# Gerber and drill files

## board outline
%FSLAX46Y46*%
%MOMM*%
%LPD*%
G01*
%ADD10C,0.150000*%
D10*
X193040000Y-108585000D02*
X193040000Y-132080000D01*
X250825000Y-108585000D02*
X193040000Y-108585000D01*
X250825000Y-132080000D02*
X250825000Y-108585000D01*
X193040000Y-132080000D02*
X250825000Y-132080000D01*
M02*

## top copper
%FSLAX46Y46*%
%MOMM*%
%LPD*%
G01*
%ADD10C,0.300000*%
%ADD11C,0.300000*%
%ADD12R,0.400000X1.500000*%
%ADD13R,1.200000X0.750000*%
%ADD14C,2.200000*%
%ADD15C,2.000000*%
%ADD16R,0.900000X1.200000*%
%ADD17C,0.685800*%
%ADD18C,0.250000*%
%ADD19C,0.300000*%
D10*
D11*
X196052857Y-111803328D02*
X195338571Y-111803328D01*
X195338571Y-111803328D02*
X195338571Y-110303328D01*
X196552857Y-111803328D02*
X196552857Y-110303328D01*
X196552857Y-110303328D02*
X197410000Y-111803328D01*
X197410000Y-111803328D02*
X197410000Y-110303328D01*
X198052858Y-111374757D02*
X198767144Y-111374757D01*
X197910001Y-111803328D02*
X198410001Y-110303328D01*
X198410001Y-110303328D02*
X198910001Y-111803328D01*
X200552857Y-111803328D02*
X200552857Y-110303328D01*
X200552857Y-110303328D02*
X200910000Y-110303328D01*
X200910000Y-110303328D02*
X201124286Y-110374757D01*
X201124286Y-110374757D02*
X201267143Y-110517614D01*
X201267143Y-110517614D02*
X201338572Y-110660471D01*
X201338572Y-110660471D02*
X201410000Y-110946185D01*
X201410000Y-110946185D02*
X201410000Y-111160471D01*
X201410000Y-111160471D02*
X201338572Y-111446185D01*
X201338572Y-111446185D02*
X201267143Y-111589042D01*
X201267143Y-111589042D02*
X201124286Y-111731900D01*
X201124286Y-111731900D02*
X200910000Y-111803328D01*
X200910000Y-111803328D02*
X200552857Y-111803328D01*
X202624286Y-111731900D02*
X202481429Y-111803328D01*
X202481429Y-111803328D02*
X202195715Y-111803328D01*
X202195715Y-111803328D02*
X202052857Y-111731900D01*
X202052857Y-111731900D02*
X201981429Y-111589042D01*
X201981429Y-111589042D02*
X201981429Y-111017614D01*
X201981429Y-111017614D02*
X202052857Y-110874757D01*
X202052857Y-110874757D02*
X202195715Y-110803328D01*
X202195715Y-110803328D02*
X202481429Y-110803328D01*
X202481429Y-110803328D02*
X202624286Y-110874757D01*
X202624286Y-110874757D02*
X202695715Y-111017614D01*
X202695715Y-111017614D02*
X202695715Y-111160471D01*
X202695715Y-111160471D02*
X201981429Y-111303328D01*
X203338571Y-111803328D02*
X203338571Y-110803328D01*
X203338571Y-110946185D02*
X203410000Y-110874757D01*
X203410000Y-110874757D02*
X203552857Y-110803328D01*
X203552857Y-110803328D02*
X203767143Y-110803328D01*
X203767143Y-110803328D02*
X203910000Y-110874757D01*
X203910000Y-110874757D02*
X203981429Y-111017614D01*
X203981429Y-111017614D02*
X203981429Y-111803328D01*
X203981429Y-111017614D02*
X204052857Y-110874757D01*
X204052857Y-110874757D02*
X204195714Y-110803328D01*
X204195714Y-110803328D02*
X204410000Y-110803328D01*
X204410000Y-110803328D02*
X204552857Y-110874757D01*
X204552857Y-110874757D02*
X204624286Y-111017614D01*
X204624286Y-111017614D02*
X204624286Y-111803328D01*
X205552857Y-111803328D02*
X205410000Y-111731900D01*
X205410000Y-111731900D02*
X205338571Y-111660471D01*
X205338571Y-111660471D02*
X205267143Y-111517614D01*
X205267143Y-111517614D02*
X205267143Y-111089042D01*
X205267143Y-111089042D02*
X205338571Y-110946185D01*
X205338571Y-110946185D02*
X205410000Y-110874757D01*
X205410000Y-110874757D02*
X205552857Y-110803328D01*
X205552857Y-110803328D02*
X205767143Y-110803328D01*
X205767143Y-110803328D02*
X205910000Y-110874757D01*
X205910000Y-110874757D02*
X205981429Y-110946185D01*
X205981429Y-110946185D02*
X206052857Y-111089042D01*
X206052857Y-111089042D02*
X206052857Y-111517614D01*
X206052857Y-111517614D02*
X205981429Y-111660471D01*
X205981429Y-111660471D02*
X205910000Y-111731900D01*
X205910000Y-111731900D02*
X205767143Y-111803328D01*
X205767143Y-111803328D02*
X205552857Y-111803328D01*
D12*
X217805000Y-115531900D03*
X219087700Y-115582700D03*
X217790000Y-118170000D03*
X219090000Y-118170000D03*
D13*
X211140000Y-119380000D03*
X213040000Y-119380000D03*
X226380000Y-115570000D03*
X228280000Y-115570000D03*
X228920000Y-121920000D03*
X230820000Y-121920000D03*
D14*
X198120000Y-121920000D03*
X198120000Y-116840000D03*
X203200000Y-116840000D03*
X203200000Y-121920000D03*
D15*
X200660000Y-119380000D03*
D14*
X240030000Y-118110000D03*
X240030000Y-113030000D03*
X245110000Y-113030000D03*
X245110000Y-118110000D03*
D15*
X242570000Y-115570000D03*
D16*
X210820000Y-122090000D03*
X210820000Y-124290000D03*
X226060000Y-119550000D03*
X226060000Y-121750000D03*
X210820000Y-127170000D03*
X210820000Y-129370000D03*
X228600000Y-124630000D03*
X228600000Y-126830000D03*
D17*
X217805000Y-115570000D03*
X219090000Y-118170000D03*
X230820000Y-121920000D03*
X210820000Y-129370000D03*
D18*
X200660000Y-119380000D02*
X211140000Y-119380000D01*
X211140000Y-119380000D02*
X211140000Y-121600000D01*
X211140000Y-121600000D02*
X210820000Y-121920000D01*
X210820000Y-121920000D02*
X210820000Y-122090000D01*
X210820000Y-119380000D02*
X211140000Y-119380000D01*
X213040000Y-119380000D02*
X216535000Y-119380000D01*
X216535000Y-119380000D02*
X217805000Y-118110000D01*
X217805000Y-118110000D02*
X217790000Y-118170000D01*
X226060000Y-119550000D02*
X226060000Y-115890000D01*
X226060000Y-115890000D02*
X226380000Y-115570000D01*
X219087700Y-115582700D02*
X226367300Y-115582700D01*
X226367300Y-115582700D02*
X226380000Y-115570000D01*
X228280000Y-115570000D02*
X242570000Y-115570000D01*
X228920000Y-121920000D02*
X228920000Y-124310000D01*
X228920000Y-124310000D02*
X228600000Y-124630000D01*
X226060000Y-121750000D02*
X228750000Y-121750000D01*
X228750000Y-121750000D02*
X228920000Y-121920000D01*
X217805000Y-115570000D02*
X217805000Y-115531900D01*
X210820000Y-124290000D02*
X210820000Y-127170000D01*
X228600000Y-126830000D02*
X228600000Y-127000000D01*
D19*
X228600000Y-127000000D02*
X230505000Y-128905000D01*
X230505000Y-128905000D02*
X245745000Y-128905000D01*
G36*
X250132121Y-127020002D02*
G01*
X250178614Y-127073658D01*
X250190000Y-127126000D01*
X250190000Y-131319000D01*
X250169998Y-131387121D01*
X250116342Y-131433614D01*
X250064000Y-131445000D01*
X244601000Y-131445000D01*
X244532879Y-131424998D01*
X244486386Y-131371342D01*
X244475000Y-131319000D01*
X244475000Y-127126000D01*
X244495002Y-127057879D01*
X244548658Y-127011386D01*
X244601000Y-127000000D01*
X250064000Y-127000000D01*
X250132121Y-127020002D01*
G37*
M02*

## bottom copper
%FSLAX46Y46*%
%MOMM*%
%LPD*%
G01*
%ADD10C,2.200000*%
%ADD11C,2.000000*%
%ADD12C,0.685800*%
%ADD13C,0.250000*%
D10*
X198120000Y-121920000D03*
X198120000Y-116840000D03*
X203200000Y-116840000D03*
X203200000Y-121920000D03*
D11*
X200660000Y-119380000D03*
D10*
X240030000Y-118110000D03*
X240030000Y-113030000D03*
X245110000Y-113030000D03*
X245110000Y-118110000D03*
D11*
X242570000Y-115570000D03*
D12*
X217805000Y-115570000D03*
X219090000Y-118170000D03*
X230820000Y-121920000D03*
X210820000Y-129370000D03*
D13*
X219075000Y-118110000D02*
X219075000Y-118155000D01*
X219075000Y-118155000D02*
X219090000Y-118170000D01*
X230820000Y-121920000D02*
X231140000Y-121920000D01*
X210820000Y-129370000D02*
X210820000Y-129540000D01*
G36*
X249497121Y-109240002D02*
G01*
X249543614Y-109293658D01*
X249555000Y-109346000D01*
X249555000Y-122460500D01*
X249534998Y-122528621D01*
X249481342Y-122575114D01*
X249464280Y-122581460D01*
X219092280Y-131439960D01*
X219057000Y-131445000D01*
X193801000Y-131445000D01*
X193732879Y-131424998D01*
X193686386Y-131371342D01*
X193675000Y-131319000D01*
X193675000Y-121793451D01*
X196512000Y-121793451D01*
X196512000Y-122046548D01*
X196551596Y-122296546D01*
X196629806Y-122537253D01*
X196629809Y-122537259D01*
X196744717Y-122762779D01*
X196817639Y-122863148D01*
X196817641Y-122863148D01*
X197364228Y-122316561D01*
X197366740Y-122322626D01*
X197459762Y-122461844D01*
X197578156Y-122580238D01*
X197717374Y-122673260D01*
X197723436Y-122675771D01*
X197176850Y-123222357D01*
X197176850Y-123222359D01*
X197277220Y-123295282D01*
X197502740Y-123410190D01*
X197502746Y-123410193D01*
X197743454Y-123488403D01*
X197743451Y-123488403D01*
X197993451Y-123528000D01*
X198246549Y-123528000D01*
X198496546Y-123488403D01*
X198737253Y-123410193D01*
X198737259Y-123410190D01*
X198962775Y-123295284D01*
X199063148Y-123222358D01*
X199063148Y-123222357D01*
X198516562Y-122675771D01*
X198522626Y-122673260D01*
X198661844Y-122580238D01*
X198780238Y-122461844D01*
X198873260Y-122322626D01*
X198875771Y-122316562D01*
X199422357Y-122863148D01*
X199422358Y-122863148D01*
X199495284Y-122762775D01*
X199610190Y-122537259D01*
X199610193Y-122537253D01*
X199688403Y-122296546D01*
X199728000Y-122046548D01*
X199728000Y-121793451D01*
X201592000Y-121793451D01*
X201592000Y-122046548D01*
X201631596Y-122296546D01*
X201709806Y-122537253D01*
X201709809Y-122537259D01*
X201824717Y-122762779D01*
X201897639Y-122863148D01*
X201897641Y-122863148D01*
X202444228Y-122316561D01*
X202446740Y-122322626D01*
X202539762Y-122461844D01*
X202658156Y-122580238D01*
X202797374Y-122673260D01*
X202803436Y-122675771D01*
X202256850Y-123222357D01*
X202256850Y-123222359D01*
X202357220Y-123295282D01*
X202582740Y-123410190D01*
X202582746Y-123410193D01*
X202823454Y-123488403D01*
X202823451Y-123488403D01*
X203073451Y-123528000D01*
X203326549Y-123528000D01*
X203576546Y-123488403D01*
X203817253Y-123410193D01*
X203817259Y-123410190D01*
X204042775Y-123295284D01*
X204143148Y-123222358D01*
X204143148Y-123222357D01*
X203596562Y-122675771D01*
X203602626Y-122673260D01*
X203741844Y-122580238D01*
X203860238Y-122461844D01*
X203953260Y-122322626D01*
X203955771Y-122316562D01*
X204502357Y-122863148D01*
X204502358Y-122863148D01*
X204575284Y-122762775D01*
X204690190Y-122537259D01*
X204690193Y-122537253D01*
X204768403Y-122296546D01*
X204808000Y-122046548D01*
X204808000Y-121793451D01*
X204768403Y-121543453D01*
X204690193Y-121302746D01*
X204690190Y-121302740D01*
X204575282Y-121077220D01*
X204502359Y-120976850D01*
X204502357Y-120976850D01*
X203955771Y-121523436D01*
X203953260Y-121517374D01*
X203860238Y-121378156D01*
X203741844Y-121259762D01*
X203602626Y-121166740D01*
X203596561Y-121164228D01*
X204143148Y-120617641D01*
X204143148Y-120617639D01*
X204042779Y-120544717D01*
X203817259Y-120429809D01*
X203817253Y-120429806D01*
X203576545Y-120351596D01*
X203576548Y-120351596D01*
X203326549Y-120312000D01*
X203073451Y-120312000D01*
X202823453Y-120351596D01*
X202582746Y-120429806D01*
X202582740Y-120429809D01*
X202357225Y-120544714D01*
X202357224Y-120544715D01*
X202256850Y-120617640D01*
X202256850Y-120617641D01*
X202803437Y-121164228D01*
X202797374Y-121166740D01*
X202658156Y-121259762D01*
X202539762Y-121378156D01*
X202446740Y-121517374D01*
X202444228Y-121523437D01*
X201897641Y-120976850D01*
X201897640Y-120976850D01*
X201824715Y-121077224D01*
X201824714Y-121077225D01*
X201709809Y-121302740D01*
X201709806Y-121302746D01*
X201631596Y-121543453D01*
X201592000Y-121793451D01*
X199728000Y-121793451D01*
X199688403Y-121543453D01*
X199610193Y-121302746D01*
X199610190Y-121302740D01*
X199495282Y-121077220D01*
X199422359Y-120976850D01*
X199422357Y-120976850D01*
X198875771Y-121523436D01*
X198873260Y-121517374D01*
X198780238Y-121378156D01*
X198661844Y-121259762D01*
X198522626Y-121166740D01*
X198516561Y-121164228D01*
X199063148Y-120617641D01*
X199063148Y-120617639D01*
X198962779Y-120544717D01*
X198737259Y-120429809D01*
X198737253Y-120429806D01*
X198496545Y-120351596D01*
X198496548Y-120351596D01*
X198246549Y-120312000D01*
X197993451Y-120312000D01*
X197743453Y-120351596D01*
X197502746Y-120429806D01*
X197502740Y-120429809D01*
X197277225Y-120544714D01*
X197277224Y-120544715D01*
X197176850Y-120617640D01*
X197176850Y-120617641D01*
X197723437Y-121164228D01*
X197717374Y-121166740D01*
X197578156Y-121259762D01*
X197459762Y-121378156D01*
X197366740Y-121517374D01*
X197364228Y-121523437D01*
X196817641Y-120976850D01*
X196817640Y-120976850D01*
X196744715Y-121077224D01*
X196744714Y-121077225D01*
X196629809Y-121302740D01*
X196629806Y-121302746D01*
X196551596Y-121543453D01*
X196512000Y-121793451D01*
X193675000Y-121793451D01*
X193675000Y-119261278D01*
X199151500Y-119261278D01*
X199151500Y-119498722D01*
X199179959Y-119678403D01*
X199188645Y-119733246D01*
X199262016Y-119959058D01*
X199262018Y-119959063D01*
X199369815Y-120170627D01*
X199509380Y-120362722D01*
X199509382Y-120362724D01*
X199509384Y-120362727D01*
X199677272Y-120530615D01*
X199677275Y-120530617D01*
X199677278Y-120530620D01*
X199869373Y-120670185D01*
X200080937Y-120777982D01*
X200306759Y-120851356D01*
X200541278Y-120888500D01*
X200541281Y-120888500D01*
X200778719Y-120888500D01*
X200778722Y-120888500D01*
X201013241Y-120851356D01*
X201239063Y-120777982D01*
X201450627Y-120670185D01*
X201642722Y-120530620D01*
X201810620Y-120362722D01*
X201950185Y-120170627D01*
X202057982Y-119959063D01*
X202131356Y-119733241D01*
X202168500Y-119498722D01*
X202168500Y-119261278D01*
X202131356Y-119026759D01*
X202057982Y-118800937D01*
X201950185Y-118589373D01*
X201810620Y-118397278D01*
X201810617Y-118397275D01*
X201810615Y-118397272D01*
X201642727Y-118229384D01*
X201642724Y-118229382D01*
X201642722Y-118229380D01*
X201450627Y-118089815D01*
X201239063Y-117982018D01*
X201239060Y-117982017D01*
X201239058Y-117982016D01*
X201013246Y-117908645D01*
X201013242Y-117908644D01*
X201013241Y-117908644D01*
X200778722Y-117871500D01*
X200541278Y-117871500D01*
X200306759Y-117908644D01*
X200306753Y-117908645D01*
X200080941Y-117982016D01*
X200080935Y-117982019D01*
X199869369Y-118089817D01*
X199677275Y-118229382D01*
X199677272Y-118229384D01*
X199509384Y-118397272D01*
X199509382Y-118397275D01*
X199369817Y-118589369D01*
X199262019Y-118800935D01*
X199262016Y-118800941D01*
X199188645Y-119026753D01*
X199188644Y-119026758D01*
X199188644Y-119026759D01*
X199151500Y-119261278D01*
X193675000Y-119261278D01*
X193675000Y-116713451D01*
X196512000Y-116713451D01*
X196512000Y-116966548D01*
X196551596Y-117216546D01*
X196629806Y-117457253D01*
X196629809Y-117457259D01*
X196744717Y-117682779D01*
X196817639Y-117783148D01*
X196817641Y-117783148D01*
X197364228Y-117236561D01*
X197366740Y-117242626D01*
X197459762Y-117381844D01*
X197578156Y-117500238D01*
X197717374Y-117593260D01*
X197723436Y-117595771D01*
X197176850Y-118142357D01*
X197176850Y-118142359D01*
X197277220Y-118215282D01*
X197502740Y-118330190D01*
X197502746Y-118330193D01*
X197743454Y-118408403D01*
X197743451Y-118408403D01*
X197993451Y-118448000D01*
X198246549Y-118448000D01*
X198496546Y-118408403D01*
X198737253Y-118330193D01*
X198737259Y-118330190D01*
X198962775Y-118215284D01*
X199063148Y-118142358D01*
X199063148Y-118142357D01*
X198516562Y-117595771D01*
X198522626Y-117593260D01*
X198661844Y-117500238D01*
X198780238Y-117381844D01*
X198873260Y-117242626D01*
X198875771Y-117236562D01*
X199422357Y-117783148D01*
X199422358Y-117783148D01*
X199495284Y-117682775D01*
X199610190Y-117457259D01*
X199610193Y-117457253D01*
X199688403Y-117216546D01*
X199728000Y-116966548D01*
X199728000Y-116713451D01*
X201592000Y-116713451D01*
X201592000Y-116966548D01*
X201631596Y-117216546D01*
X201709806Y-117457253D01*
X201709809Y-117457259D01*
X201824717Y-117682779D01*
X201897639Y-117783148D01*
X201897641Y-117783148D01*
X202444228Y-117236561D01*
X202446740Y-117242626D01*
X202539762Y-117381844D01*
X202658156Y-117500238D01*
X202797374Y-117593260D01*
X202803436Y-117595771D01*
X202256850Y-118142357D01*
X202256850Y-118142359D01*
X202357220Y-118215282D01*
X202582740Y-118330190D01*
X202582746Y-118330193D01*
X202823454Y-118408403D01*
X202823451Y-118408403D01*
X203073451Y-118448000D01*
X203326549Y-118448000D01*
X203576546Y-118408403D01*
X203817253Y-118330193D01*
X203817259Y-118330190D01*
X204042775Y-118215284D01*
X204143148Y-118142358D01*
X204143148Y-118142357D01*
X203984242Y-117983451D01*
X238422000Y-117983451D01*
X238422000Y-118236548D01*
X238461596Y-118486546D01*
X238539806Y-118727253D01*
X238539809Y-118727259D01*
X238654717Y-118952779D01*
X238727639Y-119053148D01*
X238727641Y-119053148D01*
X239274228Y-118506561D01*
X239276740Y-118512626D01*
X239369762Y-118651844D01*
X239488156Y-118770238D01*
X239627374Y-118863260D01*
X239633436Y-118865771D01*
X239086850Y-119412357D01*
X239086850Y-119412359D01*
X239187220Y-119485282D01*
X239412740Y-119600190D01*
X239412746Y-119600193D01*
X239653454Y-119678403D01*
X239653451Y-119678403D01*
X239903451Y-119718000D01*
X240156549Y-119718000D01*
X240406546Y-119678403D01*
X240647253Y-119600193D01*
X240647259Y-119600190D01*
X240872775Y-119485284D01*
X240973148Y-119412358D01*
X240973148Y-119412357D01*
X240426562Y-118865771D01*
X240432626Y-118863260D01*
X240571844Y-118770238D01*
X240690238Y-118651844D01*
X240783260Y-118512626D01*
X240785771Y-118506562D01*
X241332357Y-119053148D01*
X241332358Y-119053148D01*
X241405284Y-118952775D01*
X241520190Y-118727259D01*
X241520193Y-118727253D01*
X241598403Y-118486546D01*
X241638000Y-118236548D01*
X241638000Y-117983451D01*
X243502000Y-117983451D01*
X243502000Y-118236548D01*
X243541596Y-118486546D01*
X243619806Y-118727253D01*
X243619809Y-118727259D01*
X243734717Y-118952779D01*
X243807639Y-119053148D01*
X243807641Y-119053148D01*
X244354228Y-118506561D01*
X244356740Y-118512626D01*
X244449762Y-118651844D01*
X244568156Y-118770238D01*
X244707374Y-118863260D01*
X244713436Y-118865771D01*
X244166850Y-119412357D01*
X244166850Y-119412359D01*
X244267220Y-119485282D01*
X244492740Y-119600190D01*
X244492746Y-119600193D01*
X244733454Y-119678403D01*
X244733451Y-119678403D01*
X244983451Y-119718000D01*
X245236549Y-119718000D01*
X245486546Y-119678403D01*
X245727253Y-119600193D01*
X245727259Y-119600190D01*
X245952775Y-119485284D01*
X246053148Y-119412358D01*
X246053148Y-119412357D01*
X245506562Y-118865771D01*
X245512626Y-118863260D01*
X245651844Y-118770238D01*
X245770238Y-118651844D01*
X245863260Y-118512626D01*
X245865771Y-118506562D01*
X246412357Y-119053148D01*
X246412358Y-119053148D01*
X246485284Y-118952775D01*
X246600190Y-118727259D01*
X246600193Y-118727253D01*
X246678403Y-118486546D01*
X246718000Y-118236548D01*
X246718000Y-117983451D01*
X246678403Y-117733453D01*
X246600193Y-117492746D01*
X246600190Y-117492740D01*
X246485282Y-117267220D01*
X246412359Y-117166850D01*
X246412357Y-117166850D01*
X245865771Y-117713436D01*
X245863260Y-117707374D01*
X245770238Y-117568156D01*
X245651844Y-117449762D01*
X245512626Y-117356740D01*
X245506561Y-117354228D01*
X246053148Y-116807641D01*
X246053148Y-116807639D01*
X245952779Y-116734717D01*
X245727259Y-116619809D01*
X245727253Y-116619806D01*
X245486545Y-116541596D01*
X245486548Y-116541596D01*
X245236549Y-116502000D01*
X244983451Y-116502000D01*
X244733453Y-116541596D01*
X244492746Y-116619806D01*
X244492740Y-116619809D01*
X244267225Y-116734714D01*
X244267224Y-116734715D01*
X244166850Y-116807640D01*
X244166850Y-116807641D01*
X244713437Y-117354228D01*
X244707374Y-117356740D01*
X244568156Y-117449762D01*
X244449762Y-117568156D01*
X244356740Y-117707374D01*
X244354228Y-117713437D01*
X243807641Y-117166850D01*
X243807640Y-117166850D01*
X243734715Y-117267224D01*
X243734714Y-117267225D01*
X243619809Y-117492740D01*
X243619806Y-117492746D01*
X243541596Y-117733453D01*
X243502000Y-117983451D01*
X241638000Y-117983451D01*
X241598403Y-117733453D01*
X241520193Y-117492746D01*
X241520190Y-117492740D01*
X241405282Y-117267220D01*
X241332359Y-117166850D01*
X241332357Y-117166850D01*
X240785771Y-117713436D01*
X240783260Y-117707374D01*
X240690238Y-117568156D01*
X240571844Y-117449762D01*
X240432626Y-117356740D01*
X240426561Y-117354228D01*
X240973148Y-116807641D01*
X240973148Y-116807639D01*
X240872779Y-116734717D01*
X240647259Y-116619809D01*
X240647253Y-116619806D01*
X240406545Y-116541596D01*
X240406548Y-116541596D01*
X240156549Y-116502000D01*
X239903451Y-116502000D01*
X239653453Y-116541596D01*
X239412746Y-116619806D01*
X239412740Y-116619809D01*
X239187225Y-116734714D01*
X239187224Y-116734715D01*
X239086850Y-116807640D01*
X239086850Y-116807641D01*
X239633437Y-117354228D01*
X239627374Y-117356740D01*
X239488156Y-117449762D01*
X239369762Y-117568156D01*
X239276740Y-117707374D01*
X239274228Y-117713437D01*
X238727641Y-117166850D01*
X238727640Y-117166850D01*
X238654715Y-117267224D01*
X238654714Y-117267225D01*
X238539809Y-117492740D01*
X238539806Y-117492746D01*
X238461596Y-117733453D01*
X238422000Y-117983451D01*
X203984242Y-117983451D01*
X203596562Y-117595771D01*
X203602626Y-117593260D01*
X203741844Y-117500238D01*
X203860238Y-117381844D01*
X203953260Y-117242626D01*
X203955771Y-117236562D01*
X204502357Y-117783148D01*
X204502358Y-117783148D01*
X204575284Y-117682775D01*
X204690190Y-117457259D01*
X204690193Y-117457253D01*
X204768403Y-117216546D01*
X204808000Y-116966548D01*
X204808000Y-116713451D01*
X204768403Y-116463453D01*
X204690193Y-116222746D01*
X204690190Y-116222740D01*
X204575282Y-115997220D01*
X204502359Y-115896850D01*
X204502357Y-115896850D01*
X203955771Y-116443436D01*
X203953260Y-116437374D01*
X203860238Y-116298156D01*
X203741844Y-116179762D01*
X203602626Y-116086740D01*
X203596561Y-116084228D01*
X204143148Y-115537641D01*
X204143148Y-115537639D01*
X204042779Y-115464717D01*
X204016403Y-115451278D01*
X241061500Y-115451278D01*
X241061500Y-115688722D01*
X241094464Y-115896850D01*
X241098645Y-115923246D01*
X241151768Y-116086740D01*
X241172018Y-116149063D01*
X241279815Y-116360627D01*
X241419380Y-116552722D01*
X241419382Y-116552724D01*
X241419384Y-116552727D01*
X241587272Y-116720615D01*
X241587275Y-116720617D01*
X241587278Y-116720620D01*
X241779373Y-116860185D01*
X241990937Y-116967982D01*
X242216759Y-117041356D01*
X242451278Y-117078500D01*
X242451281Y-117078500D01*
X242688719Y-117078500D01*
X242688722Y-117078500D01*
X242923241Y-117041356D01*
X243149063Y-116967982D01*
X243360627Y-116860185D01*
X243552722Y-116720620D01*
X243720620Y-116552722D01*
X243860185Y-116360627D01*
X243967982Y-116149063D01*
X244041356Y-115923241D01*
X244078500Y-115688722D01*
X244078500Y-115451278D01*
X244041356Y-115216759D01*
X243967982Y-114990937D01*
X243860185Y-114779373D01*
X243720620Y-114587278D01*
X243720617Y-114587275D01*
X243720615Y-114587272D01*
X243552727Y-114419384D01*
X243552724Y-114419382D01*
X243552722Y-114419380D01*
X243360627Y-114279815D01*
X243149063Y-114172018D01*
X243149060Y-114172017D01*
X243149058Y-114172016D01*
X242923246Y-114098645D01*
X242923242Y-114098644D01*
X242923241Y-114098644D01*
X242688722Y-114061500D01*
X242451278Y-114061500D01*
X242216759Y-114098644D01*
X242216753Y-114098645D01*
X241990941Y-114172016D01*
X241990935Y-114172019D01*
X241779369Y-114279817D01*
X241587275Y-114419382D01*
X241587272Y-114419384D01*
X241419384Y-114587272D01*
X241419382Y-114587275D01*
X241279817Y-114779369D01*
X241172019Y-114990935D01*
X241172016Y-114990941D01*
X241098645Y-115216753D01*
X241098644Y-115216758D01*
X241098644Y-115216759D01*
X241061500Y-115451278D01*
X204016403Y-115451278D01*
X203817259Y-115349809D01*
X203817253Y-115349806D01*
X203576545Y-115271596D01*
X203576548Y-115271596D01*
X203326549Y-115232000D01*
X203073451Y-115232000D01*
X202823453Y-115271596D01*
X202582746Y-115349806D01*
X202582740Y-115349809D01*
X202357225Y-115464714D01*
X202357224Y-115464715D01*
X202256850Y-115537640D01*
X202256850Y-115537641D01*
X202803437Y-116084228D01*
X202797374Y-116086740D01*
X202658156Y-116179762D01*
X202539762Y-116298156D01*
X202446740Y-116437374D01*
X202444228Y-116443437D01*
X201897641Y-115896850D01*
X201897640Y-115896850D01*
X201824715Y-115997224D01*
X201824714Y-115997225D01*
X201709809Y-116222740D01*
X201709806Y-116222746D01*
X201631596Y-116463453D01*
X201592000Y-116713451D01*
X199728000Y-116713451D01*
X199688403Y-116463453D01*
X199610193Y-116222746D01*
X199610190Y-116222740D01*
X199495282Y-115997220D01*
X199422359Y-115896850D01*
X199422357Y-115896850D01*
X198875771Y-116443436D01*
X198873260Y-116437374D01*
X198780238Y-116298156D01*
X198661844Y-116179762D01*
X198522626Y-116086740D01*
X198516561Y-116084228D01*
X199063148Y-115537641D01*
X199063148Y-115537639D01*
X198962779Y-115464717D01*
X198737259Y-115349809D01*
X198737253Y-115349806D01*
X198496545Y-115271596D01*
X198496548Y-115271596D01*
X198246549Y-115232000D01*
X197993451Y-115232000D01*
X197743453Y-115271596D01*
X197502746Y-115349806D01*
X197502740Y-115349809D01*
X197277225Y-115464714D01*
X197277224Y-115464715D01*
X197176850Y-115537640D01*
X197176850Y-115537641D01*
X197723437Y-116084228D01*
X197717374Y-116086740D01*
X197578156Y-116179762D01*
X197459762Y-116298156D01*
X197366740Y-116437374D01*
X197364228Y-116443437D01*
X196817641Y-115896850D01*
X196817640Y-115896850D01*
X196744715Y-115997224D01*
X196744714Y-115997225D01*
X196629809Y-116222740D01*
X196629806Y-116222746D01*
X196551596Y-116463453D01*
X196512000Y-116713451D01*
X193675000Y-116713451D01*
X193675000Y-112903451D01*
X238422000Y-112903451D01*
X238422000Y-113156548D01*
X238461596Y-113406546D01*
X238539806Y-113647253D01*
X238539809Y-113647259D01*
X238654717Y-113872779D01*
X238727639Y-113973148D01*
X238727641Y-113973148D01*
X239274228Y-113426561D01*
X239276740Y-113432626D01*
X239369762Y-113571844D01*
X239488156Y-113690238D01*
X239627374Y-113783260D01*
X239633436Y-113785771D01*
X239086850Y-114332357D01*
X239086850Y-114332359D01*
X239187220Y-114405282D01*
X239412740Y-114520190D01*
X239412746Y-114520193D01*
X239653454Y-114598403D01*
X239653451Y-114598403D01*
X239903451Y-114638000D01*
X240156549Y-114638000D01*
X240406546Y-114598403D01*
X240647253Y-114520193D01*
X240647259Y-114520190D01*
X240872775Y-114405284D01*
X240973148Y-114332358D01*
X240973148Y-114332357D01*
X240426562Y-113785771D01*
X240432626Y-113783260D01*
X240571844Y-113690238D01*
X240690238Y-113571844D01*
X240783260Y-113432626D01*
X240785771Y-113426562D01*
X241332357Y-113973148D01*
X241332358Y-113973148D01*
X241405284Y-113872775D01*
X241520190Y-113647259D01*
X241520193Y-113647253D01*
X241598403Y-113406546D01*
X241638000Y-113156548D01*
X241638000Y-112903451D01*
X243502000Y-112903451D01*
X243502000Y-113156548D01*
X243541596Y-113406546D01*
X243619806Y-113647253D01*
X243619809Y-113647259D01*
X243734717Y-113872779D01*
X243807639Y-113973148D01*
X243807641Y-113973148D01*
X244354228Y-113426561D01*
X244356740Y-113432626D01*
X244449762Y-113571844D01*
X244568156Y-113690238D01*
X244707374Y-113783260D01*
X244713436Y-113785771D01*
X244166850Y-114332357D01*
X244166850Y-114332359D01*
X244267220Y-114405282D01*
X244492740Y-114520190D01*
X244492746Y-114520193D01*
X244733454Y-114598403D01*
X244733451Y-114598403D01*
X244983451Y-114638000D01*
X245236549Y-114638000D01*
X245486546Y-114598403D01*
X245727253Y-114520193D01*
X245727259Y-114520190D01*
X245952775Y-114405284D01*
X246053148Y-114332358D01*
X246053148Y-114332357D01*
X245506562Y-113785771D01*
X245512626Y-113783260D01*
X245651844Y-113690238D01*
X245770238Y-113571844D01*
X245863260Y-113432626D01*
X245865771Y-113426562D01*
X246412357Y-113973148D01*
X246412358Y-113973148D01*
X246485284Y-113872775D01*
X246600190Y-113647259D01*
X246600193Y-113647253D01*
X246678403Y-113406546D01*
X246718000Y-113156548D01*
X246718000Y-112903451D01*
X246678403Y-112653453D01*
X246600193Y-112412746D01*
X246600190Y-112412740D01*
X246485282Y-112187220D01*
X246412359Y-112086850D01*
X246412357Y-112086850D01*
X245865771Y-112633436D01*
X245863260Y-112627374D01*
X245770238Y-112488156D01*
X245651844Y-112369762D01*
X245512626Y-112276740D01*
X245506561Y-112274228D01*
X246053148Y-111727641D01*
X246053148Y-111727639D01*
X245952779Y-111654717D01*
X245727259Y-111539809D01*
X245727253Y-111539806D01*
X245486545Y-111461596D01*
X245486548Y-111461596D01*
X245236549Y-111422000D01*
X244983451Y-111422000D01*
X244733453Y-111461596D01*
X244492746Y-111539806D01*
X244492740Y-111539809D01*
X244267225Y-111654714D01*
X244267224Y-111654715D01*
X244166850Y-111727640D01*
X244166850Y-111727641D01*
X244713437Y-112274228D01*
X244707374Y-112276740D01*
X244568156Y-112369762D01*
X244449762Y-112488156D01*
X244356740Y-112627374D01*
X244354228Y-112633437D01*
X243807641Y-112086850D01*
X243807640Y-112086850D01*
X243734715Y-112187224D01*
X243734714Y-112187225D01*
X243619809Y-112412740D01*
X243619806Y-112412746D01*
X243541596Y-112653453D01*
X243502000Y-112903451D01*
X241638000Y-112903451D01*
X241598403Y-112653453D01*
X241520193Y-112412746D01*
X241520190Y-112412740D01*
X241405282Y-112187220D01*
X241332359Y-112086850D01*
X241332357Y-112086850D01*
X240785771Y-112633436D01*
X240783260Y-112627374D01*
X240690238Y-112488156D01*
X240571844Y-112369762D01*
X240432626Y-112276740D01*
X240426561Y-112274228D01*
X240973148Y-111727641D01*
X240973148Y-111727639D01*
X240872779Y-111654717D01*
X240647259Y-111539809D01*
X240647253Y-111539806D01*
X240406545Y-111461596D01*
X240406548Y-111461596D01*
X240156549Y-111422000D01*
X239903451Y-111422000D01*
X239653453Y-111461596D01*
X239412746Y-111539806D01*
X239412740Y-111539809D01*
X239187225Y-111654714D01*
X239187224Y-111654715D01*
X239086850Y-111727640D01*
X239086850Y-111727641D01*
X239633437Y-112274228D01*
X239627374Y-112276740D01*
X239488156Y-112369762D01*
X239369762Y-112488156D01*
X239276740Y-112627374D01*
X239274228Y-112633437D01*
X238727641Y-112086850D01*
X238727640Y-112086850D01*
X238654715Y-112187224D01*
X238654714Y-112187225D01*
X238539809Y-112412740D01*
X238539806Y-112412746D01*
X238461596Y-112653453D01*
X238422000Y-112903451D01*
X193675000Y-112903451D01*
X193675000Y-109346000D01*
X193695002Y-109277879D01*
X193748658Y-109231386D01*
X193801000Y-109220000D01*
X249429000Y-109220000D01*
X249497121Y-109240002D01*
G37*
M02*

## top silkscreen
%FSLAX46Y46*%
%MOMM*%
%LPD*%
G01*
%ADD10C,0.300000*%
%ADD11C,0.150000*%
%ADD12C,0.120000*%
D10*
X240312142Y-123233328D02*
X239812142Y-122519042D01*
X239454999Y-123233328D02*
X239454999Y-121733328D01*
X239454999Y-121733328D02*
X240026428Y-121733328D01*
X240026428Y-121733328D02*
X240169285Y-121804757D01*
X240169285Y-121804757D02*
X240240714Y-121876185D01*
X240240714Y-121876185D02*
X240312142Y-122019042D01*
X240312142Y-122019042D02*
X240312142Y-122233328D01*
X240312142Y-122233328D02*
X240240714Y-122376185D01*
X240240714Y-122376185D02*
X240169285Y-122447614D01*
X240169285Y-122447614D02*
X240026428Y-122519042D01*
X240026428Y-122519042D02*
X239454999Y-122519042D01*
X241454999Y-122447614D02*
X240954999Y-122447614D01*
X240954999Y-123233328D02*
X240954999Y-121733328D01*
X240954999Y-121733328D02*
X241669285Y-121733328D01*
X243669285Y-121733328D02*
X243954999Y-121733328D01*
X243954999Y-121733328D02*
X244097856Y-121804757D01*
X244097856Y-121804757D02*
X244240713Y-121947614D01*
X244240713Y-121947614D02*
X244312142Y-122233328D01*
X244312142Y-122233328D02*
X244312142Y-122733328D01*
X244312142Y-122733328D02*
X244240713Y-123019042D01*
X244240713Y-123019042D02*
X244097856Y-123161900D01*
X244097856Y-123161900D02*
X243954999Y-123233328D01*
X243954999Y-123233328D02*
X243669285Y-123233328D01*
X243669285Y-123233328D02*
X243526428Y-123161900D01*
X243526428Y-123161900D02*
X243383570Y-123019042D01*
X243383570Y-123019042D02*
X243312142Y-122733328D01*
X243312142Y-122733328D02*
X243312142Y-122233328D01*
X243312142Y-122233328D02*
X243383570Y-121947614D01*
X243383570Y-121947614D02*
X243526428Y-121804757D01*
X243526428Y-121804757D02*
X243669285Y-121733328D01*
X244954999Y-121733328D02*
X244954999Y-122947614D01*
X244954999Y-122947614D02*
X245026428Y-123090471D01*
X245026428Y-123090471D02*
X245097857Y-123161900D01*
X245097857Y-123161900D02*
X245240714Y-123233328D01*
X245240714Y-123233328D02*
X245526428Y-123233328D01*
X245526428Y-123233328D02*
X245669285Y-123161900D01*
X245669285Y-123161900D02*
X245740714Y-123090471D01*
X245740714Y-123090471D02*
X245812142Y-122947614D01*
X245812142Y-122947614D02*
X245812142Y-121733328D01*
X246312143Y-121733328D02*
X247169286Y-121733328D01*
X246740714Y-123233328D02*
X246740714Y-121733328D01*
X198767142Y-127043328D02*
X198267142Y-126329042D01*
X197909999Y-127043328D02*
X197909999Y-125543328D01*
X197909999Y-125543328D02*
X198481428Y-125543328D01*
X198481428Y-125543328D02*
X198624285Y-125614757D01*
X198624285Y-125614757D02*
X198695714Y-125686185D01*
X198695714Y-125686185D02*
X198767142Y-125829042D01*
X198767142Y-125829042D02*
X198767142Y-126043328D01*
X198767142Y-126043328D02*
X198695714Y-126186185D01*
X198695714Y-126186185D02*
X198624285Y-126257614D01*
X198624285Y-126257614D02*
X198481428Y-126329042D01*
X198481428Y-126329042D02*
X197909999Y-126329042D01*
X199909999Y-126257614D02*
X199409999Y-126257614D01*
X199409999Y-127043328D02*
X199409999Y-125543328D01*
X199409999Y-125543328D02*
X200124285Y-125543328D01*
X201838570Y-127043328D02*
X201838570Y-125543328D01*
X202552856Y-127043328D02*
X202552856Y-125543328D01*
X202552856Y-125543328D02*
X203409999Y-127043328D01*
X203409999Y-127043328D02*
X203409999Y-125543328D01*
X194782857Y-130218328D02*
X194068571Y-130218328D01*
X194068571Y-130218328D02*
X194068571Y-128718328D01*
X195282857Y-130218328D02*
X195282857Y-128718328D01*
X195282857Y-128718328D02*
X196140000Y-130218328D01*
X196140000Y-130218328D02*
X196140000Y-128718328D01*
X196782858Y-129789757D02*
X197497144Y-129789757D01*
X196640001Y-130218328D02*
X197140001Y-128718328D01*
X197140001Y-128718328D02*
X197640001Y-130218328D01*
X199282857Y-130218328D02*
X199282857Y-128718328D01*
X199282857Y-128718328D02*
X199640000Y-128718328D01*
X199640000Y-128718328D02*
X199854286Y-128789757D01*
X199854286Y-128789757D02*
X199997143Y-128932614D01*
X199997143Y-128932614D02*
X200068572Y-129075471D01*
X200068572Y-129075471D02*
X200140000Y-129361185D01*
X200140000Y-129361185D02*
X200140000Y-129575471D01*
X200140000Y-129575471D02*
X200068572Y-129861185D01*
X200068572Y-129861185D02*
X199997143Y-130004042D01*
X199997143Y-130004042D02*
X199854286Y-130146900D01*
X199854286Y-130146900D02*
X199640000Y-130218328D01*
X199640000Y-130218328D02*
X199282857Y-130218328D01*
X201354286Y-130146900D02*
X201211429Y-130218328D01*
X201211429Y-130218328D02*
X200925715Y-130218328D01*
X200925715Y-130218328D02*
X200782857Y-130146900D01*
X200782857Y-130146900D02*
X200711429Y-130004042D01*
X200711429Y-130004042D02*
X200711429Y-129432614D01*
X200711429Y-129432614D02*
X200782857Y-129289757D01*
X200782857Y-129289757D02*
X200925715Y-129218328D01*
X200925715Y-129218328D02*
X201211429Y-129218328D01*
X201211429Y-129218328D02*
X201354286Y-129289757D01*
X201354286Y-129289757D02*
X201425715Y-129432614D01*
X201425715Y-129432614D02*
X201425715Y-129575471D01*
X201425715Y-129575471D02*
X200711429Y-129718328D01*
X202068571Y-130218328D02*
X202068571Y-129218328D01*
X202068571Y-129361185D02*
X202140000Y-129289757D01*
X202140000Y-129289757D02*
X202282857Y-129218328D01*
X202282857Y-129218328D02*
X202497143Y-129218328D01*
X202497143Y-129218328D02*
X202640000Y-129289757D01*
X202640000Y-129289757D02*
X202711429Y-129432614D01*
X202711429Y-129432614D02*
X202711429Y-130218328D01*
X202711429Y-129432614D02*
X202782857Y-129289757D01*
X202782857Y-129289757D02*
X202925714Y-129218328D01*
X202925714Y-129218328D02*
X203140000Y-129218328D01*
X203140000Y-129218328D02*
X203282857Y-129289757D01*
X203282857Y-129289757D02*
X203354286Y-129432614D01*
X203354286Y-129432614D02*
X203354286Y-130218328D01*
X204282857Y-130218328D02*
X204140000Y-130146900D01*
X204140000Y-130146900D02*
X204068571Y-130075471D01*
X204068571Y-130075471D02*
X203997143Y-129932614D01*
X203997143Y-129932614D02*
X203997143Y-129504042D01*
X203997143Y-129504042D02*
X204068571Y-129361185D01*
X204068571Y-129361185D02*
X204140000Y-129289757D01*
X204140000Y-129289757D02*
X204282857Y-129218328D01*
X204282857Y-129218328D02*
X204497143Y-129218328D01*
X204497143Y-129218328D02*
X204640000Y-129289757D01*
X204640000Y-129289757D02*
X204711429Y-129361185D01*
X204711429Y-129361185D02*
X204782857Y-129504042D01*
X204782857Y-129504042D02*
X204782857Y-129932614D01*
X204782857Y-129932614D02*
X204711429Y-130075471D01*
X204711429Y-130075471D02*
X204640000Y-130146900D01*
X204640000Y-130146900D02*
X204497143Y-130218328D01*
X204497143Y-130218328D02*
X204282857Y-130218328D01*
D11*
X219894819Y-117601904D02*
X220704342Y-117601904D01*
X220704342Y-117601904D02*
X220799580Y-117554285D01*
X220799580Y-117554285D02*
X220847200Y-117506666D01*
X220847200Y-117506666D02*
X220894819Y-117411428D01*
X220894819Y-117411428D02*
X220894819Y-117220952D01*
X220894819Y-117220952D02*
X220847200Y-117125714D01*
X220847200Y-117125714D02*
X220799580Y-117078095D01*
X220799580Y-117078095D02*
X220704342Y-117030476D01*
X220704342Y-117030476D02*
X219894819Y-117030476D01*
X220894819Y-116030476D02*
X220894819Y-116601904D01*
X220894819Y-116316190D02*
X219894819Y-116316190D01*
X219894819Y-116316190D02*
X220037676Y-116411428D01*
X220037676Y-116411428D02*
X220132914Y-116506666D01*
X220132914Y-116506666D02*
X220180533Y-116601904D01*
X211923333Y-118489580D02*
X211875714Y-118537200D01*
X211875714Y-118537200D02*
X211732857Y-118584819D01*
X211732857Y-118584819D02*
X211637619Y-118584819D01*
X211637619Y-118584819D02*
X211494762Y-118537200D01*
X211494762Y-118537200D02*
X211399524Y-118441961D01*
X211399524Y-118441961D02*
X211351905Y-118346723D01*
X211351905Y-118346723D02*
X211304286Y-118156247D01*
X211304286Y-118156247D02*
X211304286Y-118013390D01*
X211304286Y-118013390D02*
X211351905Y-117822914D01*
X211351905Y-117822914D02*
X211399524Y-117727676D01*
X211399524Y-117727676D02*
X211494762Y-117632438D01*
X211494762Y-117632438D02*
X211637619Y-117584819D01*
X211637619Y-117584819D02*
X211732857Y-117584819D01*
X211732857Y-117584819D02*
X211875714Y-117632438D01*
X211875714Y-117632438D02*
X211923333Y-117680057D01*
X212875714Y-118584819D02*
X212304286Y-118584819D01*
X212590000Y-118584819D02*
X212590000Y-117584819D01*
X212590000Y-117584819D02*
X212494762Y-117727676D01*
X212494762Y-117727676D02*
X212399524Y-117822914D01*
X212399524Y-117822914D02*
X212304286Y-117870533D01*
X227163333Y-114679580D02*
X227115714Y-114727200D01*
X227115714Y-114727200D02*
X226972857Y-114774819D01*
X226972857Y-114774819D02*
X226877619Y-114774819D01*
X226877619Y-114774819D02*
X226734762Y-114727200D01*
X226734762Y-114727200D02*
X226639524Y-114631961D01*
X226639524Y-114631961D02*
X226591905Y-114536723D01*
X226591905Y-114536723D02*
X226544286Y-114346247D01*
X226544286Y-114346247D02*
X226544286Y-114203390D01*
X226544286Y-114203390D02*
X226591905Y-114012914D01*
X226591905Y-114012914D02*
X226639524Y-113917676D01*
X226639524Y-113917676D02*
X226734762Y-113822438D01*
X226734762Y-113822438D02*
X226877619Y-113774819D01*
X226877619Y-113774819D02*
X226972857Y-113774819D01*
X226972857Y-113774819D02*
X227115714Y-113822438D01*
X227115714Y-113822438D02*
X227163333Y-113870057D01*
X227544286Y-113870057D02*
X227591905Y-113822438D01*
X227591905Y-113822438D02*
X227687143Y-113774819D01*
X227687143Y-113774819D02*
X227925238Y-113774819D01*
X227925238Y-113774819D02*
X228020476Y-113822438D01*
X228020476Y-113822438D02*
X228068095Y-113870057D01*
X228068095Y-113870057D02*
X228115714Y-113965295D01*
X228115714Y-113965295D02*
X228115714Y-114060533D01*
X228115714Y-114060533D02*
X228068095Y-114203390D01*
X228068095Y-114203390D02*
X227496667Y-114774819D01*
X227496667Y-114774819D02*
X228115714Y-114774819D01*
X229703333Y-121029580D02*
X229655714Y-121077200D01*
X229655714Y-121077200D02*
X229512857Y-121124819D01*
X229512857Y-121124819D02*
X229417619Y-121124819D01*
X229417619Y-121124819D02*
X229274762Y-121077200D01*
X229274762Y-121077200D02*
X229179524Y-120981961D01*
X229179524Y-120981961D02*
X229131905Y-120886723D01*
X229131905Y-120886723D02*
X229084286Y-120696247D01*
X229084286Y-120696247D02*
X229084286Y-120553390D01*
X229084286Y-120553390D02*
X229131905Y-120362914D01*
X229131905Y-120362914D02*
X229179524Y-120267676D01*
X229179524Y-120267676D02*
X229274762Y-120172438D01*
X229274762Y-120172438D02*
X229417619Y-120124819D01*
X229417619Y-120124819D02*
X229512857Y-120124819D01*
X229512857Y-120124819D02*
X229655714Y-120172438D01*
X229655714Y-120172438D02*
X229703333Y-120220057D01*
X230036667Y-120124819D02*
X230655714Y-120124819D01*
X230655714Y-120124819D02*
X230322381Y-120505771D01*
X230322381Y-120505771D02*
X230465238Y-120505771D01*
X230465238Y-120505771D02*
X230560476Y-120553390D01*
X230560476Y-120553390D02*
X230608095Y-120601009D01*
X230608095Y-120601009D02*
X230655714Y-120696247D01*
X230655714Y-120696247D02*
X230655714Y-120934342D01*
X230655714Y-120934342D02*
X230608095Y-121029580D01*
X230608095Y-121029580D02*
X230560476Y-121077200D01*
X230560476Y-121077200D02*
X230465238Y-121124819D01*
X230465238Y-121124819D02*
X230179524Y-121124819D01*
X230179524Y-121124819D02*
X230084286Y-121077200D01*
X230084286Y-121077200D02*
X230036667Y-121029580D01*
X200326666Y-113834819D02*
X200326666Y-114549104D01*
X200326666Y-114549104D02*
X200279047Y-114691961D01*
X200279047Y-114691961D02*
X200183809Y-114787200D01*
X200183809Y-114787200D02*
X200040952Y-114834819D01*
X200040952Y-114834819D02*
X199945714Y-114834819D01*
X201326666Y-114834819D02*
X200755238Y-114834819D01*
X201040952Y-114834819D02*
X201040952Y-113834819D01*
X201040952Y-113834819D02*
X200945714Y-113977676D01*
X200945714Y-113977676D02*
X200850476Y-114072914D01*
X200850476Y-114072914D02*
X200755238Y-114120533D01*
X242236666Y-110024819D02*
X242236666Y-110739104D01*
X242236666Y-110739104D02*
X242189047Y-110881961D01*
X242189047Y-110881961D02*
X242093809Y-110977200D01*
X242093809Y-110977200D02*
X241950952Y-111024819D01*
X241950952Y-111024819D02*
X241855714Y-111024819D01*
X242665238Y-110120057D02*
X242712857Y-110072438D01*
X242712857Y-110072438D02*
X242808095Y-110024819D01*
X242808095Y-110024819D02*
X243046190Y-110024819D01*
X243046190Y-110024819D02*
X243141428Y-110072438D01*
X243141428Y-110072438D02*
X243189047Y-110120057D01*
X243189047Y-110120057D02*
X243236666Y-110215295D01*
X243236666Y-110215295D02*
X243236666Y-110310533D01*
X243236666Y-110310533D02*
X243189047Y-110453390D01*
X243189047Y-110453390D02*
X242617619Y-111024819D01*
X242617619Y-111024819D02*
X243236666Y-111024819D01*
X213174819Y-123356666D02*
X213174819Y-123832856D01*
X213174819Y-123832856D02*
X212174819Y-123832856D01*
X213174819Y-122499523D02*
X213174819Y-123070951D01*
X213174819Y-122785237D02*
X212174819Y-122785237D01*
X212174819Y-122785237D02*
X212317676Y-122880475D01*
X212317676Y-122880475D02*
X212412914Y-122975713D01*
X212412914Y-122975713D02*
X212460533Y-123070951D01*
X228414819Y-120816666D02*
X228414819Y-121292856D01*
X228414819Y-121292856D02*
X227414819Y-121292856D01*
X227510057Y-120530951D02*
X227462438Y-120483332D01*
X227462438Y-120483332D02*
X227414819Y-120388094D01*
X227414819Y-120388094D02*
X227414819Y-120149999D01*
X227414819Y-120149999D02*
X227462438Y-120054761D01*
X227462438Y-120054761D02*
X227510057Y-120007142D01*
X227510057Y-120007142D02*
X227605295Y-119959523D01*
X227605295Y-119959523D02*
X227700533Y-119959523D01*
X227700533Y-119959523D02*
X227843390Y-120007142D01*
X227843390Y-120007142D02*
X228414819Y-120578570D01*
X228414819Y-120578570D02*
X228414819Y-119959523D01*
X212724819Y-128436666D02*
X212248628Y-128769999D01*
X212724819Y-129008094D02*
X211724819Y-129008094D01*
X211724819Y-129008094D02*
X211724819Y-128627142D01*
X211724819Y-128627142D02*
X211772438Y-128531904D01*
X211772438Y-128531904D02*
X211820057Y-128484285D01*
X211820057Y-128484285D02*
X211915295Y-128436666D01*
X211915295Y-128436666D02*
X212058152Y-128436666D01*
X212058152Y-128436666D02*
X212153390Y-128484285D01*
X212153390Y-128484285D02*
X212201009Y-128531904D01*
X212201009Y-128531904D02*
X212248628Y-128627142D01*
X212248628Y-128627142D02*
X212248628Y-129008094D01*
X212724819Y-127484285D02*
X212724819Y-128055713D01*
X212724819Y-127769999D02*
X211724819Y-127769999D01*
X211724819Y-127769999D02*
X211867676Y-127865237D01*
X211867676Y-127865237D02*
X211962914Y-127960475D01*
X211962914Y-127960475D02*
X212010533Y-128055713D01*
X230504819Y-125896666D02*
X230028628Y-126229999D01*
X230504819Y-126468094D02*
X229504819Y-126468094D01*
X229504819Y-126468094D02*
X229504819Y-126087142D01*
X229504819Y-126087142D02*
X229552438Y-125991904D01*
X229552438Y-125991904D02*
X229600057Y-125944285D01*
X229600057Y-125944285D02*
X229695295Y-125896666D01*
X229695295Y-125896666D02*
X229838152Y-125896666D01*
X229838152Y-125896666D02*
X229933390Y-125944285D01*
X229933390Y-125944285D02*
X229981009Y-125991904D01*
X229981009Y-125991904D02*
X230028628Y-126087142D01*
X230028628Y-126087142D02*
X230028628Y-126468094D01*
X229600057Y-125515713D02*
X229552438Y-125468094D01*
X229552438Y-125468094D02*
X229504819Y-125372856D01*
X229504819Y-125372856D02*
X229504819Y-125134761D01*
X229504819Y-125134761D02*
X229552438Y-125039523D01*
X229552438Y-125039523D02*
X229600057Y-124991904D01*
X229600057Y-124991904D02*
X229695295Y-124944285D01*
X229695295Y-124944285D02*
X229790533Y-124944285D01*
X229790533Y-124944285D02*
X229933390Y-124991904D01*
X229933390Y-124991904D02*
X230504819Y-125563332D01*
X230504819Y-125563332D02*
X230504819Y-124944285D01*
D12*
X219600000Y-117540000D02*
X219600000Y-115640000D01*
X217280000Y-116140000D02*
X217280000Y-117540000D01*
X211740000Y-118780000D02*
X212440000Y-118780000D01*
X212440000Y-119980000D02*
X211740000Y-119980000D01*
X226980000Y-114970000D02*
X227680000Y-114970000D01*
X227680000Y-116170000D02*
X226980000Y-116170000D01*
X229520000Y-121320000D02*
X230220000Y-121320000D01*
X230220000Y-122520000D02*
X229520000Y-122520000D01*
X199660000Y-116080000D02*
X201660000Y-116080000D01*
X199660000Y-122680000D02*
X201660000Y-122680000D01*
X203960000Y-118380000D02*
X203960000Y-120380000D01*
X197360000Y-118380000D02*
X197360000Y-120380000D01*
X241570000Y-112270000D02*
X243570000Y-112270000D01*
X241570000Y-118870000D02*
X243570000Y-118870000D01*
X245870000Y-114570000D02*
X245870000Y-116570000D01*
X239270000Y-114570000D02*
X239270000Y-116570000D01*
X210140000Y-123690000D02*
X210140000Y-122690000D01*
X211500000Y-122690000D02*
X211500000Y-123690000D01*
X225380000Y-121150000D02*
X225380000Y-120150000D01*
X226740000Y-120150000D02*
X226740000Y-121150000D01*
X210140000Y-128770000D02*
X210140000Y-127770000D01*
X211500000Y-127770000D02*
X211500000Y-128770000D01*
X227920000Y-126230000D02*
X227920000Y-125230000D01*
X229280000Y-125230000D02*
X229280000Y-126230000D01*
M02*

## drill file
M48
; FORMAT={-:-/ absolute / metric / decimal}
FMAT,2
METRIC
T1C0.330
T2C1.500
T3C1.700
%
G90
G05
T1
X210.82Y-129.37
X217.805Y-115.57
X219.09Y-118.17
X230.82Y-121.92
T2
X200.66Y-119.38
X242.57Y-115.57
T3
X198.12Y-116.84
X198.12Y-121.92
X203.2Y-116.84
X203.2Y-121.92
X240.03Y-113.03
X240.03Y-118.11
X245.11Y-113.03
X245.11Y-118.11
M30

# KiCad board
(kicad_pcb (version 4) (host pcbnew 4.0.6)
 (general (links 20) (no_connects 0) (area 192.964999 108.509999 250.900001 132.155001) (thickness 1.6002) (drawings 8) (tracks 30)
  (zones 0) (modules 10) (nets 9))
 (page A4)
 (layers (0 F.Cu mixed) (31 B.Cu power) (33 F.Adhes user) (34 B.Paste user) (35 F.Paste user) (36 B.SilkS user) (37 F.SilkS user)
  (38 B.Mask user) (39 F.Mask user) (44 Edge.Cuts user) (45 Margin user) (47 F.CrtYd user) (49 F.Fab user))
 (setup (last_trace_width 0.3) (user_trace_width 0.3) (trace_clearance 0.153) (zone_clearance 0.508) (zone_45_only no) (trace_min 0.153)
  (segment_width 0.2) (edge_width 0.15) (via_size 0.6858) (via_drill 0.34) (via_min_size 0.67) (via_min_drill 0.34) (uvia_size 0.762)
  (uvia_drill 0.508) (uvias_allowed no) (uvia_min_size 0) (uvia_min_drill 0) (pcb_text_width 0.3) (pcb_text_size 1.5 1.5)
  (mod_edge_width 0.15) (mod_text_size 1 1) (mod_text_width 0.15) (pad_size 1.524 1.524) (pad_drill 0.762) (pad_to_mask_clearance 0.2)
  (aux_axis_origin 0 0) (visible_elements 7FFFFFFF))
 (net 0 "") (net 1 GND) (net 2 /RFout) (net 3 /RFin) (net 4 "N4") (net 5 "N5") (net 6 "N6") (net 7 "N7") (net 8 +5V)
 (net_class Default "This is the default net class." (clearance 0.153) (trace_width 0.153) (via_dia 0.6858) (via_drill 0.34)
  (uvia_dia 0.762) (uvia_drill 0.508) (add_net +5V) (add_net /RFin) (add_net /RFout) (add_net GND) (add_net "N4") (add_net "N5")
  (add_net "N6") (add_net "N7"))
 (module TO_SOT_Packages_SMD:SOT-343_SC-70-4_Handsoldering (layer F.Cu) (at 218.44 116.84 270)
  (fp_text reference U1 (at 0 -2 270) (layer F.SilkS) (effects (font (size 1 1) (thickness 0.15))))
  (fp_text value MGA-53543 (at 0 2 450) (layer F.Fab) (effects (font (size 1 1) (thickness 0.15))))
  (fp_line (start 0.7 -1.16) (end -1.2 -1.16) (layer F.SilkS) (width 0.12))
  (fp_line (start -0.7 1.16) (end 0.7 1.16) (layer F.SilkS) (width 0.12))
  (pad 1 smd rect (at -1.3081 0.635 270) (size 1.5 0.4) (layers F.Cu F.Paste F.Mask) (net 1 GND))
  (pad 2 smd rect (at -1.2573 -0.6477 270) (size 1.5 0.4) (layers F.Cu F.Paste F.Mask) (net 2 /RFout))
  (pad 3 smd rect (at 1.33 0.65 270) (size 1.5 0.4) (layers F.Cu F.Paste F.Mask) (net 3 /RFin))
  (pad 4 smd rect (at 1.33 -0.65 270) (size 1.5 0.4) (layers F.Cu F.Paste F.Mask) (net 1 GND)))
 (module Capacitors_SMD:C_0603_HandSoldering (layer F.Cu) (at 212.09 119.38)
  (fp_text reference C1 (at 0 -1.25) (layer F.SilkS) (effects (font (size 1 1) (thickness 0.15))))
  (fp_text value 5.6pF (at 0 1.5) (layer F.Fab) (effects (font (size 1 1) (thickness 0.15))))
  (fp_line (start -0.35 -0.6) (end 0.35 -0.6) (layer F.SilkS) (width 0.12))
  (fp_line (start 0.35 0.6) (end -0.35 0.6) (layer F.SilkS) (width 0.12))
  (pad 1 smd rect (at -0.95 0) (size 1.2 0.75) (layers F.Cu F.Paste F.Mask) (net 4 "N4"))
  (pad 2 smd rect (at 0.95 0) (size 1.2 0.75) (layers F.Cu F.Paste F.Mask) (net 3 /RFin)))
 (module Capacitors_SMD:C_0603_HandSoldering (layer F.Cu) (at 227.33 115.57)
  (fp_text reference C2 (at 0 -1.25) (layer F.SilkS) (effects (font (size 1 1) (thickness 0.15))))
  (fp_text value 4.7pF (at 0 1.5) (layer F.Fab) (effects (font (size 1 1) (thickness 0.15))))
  (fp_line (start -0.35 -0.6) (end 0.35 -0.6) (layer F.SilkS) (width 0.12))
  (fp_line (start 0.35 0.6) (end -0.35 0.6) (layer F.SilkS) (width 0.12))
  (pad 1 smd rect (at -0.95 0) (size 1.2 0.75) (layers F.Cu F.Paste F.Mask) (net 2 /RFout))
  (pad 2 smd rect (at 0.95 0) (size 1.2 0.75) (layers F.Cu F.Paste F.Mask) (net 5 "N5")))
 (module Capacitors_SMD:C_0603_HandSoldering (layer F.Cu) (at 229.87 121.92)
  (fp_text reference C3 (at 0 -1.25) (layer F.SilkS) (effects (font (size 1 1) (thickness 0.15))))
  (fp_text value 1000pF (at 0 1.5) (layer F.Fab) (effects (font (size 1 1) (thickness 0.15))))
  (fp_line (start -0.35 -0.6) (end 0.35 -0.6) (layer F.SilkS) (width 0.12))
  (fp_line (start 0.35 0.6) (end -0.35 0.6) (layer F.SilkS) (width 0.12))
  (pad 1 smd rect (at -0.95 0) (size 1.2 0.75) (layers F.Cu F.Paste F.Mask) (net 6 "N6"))
  (pad 2 smd rect (at 0.95 0) (size 1.2 0.75) (layers F.Cu F.Paste F.Mask) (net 1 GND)))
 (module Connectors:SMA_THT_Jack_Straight (layer F.Cu) (at 200.66 119.38)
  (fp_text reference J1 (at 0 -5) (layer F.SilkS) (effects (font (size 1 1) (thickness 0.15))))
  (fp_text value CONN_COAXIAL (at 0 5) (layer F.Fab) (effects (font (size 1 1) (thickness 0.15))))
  (fp_line (start -1 -3.3) (end 1 -3.3) (layer F.SilkS) (width 0.12))
  (fp_line (start -1 3.3) (end 1 3.3) (layer F.SilkS) (width 0.12))
  (fp_line (start 3.3 -1) (end 3.3 1) (layer F.SilkS) (width 0.12))
  (fp_line (start -3.3 -1) (end -3.3 1) (layer F.SilkS) (width 0.12))
  (pad 2 thru_hole circle (at -2.54 2.54) (size 2.2 2.2) (drill 1.7) (layers *.Cu *.Mask) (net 1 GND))
  (pad 2 thru_hole circle (at -2.54 -2.54) (size 2.2 2.2) (drill 1.7) (layers *.Cu *.Mask) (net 1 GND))
  (pad 2 thru_hole circle (at 2.54 -2.54) (size 2.2 2.2) (drill 1.7) (layers *.Cu *.Mask) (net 1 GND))
  (pad 2 thru_hole circle (at 2.54 2.54) (size 2.2 2.2) (drill 1.7) (layers *.Cu *.Mask) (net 1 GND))
  (pad 1 thru_hole circle (at 0 0) (size 2 2) (drill 1.5) (layers *.Cu *.Mask) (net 4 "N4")))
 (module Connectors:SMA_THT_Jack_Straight (layer F.Cu) (at 242.57 115.57)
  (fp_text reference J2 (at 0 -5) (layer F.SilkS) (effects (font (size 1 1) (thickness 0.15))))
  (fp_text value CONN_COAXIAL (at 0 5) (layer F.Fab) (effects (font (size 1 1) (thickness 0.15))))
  (fp_line (start -1 -3.3) (end 1 -3.3) (layer F.SilkS) (width 0.12))
  (fp_line (start -1 3.3) (end 1 3.3) (layer F.SilkS) (width 0.12))
  (fp_line (start 3.3 -1) (end 3.3 1) (layer F.SilkS) (width 0.12))
  (fp_line (start -3.3 -1) (end -3.3 1) (layer F.SilkS) (width 0.12))
  (pad 2 thru_hole circle (at -2.54 2.54) (size 2.2 2.2) (drill 1.7) (layers *.Cu *.Mask) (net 1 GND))
  (pad 2 thru_hole circle (at -2.54 -2.54) (size 2.2 2.2) (drill 1.7) (layers *.Cu *.Mask) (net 1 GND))
  (pad 2 thru_hole circle (at 2.54 -2.54) (size 2.2 2.2) (drill 1.7) (layers *.Cu *.Mask) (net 1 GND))
  (pad 2 thru_hole circle (at 2.54 2.54) (size 2.2 2.2) (drill 1.7) (layers *.Cu *.Mask) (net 1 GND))
  (pad 1 thru_hole circle (at 0 0) (size 2 2) (drill 1.5) (layers *.Cu *.Mask) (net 5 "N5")))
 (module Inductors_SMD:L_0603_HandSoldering (layer F.Cu) (at 210.82 123.19 270)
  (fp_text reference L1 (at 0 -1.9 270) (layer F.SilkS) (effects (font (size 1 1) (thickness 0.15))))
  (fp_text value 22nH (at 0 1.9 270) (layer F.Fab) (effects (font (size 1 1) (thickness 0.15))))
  (fp_line (start 0.5 0.68) (end -0.5 0.68) (layer F.SilkS) (width 0.12))
  (fp_line (start -0.5 -0.68) (end 0.5 -0.68) (layer F.SilkS) (width 0.12))
  (pad 1 smd rect (at -1.1 0 270) (size 1.2 0.9) (layers F.Cu F.Paste F.Mask) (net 4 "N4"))
  (pad 2 smd rect (at 1.1 0 270) (size 1.2 0.9) (layers F.Cu F.Paste F.Mask) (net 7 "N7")))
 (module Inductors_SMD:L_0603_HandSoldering (layer F.Cu) (at 226.06 120.65 270)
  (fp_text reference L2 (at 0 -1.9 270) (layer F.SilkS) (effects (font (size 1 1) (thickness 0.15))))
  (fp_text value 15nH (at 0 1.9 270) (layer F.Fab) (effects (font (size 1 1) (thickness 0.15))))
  (fp_line (start 0.5 0.68) (end -0.5 0.68) (layer F.SilkS) (width 0.12))
  (fp_line (start -0.5 -0.68) (end 0.5 -0.68) (layer F.SilkS) (width 0.12))
  (pad 1 smd rect (at -1.1 0 270) (size 1.2 0.9) (layers F.Cu F.Paste F.Mask) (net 2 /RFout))
  (pad 2 smd rect (at 1.1 0 270) (size 1.2 0.9) (layers F.Cu F.Paste F.Mask) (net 6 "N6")))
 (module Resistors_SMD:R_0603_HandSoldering (layer F.Cu) (at 210.82 128.27 270)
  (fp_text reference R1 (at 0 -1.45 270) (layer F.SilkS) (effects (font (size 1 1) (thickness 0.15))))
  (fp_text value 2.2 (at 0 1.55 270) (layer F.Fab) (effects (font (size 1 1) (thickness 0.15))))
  (fp_line (start 0.5 0.68) (end -0.5 0.68) (layer F.SilkS) (width 0.12))
  (fp_line (start -0.5 -0.68) (end 0.5 -0.68) (layer F.SilkS) (width 0.12))
  (pad 1 smd rect (at -1.1 0 270) (size 1.2 0.9) (layers F.Cu F.Paste F.Mask) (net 7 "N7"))
  (pad 2 smd rect (at 1.1 0 270) (size 1.2 0.9) (layers F.Cu F.Paste F.Mask) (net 1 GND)))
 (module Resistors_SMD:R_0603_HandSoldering (layer F.Cu) (at 228.6 125.73 270)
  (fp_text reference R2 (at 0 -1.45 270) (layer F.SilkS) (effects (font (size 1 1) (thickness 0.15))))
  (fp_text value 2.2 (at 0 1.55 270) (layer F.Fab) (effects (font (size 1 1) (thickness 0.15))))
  (fp_line (start 0.5 0.68) (end -0.5 0.68) (layer F.SilkS) (width 0.12))
  (fp_line (start -0.5 -0.68) (end 0.5 -0.68) (layer F.SilkS) (width 0.12))
  (pad 1 smd rect (at -1.1 0 270) (size 1.2 0.9) (layers F.Cu F.Paste F.Mask) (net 6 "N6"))
  (pad 2 smd rect (at 1.1 0 270) (size 1.2 0.9) (layers F.Cu F.Paste F.Mask) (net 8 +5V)))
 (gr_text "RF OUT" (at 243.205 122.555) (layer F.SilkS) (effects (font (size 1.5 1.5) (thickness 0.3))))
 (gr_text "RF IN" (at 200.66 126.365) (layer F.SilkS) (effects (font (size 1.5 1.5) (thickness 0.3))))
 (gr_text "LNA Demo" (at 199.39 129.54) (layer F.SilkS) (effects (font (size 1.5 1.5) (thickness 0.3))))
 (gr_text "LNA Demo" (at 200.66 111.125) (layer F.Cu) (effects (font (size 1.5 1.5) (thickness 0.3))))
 (gr_line (start 193.04 108.585) (end 193.04 132.08) (angle 90) (layer Edge.Cuts) (width 0.15))
 (gr_line (start 250.825 108.585) (end 193.04 108.585) (angle 90) (layer Edge.Cuts) (width 0.15))
 (gr_line (start 250.825 132.08) (end 250.825 108.585) (angle 90) (layer Edge.Cuts) (width 0.15))
 (gr_line (start 193.04 132.08) (end 250.825 132.08) (angle 90) (layer Edge.Cuts) (width 0.15))
 (segment (start 200.66 119.38) (end 211.14 119.38) (width 0.25) (layer F.Cu) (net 4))
 (segment (start 211.14 119.38) (end 211.14 121.6) (width 0.25) (layer F.Cu) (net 4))
 (segment (start 211.14 121.6) (end 210.82 121.92) (width 0.25) (layer F.Cu) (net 4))
 (segment (start 210.82 121.92) (end 210.82 122.09) (width 0.25) (layer F.Cu) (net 4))
 (segment (start 210.82 119.38) (end 211.14 119.38) (width 0.25) (layer F.Cu) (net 4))
 (segment (start 213.04 119.38) (end 216.535 119.38) (width 0.25) (layer F.Cu) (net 3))
 (segment (start 216.535 119.38) (end 217.805 118.11) (width 0.25) (layer F.Cu) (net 3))
 (segment (start 217.805 118.11) (end 217.79 118.17) (width 0.25) (layer F.Cu) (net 3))
 (segment (start 226.06 119.55) (end 226.06 115.89) (width 0.25) (layer F.Cu) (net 2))
 (segment (start 226.06 115.89) (end 226.38 115.57) (width 0.25) (layer F.Cu) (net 2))
 (segment (start 219.0877 115.5827) (end 226.3673 115.5827) (width 0.25) (layer F.Cu) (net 2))
 (segment (start 226.3673 115.5827) (end 226.38 115.57) (width 0.25) (layer F.Cu) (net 2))
 (segment (start 228.28 115.57) (end 242.57 115.57) (width 0.25) (layer F.Cu) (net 5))
 (segment (start 228.92 121.92) (end 228.92 124.31) (width 0.25) (layer F.Cu) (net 6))
 (segment (start 228.92 124.31) (end 228.6 124.63) (width 0.25) (layer F.Cu) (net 6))
 (segment (start 226.06 121.75) (end 228.75 121.75) (width 0.25) (layer F.Cu) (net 6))
 (segment (start 228.75 121.75) (end 228.92 121.92) (width 0.25) (layer F.Cu) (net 6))
 (via (at 217.805 115.57) (size 0.6858) (drill 0.3302) (layers F.Cu B.Cu) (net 1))
 (segment (start 217.805 115.57) (end 217.805 115.5319) (width 0.25) (layer F.Cu) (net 1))
 (via (at 219.09 118.17) (size 0.6858) (drill 0.3302) (layers F.Cu B.Cu) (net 1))
 (segment (start 219.075 118.11) (end 219.075 118.155) (width 0.25) (layer B.Cu) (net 1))
 (segment (start 219.075 118.155) (end 219.09 118.17) (width 0.25) (layer B.Cu) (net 1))
 (via (at 230.82 121.92) (size 0.6858) (drill 0.3302) (layers F.Cu B.Cu) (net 1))
 (segment (start 230.82 121.92) (end 231.14 121.92) (width 0.25) (layer B.Cu) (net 1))
 (via (at 210.82 129.37) (size 0.6858) (drill 0.3302) (layers F.Cu B.Cu) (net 1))
 (segment (start 210.82 129.37) (end 210.82 129.54) (width 0.25) (layer B.Cu) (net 1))
 (segment (start 210.82 124.29) (end 210.82 127.17) (width 0.25) (layer F.Cu) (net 7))
 (segment (start 228.6 126.83) (end 228.6 127) (width 0.25) (layer F.Cu) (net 8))
 (segment (start 228.6 127) (end 230.505 128.905) (width 0.3) (layer F.Cu) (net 8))
 (segment (start 230.505 128.905) (end 245.745 128.905) (width 0.3) (layer F.Cu) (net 8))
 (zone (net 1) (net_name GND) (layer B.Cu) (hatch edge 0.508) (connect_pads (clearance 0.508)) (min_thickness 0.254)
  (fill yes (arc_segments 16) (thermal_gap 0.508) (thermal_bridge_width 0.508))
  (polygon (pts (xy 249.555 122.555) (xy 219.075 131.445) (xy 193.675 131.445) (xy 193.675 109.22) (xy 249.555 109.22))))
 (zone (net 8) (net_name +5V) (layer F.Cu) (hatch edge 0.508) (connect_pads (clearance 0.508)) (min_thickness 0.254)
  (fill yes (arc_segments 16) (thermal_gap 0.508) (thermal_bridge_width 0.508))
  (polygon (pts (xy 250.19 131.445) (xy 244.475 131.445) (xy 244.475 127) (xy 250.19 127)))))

